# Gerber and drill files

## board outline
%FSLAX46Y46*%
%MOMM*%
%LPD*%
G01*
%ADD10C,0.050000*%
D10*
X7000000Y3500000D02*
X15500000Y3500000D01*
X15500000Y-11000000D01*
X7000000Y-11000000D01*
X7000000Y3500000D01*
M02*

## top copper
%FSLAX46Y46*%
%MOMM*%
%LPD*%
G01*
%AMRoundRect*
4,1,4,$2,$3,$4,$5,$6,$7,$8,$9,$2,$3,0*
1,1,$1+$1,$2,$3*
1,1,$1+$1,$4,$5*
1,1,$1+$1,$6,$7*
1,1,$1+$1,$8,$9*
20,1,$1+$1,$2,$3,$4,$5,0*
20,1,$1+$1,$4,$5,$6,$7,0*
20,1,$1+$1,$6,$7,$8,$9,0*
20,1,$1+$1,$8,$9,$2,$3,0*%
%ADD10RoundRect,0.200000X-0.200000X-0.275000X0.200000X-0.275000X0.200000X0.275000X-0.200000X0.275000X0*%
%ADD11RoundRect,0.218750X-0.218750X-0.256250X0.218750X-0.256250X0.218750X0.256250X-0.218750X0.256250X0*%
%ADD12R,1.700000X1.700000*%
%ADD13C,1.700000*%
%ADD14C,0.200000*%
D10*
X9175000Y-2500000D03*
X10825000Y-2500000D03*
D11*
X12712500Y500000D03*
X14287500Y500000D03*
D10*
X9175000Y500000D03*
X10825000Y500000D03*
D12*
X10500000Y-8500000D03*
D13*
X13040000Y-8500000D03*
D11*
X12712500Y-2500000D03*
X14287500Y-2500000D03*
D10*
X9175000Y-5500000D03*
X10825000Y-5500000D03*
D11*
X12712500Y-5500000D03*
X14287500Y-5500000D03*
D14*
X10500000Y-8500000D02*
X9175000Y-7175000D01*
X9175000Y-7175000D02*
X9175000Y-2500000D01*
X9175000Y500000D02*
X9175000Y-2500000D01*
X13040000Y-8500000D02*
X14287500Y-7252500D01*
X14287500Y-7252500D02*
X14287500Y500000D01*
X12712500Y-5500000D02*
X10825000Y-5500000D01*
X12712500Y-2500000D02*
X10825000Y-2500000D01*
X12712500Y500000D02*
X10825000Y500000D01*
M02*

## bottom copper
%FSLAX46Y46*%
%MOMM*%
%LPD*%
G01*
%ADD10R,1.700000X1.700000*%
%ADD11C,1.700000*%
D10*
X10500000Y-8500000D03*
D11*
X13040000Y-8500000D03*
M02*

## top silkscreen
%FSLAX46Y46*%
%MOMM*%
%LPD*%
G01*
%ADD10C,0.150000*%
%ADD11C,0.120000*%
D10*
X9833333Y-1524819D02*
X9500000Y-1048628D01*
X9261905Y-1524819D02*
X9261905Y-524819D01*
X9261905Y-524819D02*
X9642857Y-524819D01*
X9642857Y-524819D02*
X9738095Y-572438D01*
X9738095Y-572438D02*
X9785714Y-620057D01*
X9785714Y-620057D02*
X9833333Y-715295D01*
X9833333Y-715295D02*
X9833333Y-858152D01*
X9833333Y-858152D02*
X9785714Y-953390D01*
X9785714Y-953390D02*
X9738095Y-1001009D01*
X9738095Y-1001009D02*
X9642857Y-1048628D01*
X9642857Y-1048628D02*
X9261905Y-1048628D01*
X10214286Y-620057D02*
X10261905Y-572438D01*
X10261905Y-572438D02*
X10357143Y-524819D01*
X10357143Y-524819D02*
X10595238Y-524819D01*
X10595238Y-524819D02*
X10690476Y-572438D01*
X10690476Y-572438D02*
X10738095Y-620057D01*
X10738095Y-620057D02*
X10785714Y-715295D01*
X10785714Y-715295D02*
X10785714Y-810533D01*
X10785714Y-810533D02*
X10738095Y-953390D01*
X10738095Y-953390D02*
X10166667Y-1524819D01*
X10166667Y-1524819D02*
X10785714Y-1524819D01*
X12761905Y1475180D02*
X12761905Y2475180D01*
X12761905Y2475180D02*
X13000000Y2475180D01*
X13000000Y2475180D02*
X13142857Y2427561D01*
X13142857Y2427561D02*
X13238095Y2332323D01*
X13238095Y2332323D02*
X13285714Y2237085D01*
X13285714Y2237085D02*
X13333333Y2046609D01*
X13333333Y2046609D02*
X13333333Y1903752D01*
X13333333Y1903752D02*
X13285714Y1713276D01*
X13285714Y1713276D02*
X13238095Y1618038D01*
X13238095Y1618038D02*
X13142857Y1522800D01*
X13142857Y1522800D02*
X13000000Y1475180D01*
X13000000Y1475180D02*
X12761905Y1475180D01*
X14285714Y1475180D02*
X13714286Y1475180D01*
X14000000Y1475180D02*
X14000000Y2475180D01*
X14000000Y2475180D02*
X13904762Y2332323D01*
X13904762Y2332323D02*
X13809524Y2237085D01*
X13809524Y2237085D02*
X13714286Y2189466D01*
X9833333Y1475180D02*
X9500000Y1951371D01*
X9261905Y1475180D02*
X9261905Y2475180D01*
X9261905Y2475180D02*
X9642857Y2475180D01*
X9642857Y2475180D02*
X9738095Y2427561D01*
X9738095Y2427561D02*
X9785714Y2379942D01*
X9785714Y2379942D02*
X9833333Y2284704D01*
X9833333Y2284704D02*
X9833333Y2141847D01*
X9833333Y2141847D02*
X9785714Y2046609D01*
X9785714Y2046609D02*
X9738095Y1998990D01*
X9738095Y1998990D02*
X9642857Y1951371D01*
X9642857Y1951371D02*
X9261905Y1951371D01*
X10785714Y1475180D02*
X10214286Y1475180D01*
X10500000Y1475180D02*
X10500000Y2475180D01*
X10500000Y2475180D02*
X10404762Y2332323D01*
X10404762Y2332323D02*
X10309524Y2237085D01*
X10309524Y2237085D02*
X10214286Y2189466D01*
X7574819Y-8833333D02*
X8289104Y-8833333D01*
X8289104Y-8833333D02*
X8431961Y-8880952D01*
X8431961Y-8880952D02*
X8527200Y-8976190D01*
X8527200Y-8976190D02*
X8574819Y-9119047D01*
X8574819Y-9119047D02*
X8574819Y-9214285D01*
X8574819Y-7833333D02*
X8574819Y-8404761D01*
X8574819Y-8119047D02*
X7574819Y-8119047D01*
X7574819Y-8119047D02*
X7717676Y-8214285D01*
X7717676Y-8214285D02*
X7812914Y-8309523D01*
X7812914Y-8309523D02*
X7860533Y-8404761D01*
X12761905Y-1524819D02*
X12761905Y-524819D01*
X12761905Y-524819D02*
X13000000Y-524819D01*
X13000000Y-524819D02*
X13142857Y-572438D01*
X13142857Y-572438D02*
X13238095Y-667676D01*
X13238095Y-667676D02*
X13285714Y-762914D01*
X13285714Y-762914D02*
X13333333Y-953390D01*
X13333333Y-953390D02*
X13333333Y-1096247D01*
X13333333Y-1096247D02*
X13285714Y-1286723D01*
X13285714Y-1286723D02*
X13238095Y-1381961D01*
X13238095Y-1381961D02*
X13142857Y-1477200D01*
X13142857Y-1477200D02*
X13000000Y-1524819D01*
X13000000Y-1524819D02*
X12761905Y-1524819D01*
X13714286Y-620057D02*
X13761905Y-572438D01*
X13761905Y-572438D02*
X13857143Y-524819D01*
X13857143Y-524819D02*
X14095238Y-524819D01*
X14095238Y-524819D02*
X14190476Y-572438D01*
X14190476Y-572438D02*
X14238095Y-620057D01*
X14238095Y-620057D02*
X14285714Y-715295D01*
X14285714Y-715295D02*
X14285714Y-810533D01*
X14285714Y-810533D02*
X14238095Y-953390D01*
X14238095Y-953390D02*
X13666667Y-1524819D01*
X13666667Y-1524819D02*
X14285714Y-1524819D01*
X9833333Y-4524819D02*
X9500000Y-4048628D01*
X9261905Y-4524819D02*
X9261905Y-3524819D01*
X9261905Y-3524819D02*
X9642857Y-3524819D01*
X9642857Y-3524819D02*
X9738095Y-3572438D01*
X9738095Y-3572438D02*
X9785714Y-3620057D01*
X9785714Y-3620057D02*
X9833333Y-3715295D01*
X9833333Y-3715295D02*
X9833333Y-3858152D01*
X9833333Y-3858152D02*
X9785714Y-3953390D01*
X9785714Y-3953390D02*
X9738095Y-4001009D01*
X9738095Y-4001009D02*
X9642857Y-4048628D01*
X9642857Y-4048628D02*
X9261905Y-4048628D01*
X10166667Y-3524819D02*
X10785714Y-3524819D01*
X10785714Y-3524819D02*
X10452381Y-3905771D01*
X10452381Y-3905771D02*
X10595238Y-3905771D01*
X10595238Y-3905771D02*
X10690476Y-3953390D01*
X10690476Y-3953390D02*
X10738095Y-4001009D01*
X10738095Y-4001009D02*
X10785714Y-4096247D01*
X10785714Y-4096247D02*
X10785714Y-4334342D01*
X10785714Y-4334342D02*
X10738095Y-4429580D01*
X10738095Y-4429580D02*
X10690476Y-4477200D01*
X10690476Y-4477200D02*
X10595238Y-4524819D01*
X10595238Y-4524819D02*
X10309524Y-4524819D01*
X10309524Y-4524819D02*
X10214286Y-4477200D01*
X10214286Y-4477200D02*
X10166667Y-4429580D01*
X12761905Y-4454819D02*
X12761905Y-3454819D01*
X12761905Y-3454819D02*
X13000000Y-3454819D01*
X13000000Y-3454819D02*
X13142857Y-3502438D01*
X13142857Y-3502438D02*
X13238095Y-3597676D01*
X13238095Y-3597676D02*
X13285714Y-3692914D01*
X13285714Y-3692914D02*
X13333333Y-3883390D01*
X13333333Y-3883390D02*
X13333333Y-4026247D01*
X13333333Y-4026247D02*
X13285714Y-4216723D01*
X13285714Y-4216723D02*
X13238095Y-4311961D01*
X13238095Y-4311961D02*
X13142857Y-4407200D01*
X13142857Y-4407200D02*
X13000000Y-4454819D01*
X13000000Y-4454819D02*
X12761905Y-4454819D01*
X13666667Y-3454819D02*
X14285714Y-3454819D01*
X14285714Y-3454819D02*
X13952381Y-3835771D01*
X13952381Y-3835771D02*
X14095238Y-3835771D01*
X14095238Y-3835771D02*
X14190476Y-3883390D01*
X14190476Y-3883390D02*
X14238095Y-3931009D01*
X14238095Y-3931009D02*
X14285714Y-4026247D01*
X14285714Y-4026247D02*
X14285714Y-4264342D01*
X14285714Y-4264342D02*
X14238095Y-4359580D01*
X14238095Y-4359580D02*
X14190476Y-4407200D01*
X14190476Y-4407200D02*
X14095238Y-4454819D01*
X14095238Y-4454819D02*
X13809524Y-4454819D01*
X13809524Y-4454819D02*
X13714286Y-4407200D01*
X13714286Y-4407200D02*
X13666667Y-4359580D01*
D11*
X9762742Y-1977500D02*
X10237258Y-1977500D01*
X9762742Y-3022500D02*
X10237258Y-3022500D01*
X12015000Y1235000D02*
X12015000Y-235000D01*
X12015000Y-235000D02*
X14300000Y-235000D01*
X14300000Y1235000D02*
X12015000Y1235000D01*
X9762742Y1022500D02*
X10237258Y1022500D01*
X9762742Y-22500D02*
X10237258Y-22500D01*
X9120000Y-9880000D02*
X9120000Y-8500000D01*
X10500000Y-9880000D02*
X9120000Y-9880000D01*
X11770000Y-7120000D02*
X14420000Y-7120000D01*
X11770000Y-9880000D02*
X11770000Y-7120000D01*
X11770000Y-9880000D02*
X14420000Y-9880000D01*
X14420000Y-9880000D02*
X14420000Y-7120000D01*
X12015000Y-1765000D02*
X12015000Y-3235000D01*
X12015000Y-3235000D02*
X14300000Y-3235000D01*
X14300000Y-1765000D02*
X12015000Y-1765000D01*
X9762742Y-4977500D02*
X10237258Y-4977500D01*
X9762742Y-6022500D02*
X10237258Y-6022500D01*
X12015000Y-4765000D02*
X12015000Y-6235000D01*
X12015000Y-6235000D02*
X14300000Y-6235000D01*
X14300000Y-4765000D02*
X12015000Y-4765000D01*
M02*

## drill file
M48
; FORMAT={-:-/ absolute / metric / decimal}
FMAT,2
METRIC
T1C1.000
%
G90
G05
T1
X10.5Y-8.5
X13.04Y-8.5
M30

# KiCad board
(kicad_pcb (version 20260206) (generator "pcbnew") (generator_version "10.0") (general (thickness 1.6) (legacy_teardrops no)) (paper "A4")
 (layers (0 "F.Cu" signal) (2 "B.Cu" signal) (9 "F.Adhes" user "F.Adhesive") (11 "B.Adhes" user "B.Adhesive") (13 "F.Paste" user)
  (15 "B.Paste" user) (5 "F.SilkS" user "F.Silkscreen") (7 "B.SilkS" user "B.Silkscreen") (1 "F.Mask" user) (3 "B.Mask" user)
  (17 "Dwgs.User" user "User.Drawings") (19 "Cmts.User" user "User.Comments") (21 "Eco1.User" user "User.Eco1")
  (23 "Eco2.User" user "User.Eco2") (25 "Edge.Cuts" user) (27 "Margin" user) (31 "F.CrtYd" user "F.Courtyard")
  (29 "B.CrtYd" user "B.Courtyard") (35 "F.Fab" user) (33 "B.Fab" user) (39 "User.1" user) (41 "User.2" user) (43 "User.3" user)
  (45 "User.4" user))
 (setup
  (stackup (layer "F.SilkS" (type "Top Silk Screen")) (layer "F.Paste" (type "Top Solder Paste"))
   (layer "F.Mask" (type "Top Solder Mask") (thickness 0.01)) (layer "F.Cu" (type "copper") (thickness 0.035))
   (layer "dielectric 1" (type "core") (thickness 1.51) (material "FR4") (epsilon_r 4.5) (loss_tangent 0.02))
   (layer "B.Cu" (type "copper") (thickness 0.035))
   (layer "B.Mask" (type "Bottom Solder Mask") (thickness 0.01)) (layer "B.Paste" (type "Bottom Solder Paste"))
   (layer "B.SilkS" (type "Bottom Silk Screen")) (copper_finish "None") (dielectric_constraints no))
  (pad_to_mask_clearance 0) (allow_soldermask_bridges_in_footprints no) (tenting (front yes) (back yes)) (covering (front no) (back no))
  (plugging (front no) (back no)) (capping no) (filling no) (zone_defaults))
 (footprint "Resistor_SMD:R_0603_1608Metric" (layer "F.Cu") (at 10 2.5)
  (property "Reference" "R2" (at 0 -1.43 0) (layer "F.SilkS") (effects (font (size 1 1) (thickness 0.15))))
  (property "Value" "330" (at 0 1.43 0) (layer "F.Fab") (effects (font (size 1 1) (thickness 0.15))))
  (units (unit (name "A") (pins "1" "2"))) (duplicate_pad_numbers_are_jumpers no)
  (fp_line (start -0.237258 -0.5225) (end 0.237258 -0.5225) (stroke (width 0.12) (type solid)) (layer "F.SilkS"))
  (fp_line (start -0.237258 0.5225) (end 0.237258 0.5225) (stroke (width 0.12) (type solid)) (layer "F.SilkS"))
  (pad "1" smd roundrect (at -0.825 0) (size 0.8 0.95) (layers "F.Cu" "F.Mask" "F.Paste") (roundrect_rratio 0.25) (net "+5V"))
  (pad "2" smd roundrect (at 0.825 0) (size 0.8 0.95) (layers "F.Cu" "F.Mask" "F.Paste") (roundrect_rratio 0.25) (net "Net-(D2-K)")))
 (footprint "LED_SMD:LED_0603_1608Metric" (layer "F.Cu") (at 13.5 -0.5)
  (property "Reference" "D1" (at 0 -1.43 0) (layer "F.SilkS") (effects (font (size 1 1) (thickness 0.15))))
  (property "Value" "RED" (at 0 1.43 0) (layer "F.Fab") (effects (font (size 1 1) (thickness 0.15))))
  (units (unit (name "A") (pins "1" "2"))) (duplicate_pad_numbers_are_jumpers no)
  (fp_line (start -1.485 -0.735) (end -1.485 0.735) (stroke (width 0.12) (type solid)) (layer "F.SilkS"))
  (fp_line (start -1.485 0.735) (end 0.8 0.735) (stroke (width 0.12) (type solid)) (layer "F.SilkS"))
  (fp_line (start 0.8 -0.735) (end -1.485 -0.735) (stroke (width 0.12) (type solid)) (layer "F.SilkS"))
  (pad "1" smd roundrect (at -0.7875 0) (size 0.875 0.95) (layers "F.Cu" "F.Mask" "F.Paste") (roundrect_rratio 0.25) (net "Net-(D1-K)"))
  (pad "2" smd roundrect (at 0.7875 0) (size 0.875 0.95) (layers "F.Cu" "F.Mask" "F.Paste") (roundrect_rratio 0.25) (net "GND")))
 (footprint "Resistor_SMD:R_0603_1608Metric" (layer "F.Cu") (at 10 -0.5)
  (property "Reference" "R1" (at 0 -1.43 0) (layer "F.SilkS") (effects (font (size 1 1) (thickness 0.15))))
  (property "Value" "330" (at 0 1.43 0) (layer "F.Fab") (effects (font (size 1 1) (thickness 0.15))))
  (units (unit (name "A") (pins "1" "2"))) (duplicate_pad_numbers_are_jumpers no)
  (fp_line (start -0.237258 -0.5225) (end 0.237258 -0.5225) (stroke (width 0.12) (type solid)) (layer "F.SilkS"))
  (fp_line (start -0.237258 0.5225) (end 0.237258 0.5225) (stroke (width 0.12) (type solid)) (layer "F.SilkS"))
  (pad "1" smd roundrect (at -0.825 0) (size 0.8 0.95) (layers "F.Cu" "F.Mask" "F.Paste") (roundrect_rratio 0.25) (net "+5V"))
  (pad "2" smd roundrect (at 0.825 0) (size 0.8 0.95) (layers "F.Cu" "F.Mask" "F.Paste") (roundrect_rratio 0.25) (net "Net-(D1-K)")))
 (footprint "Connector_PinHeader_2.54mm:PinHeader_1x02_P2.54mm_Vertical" (layer "F.Cu") (at 10.5 8.5 90)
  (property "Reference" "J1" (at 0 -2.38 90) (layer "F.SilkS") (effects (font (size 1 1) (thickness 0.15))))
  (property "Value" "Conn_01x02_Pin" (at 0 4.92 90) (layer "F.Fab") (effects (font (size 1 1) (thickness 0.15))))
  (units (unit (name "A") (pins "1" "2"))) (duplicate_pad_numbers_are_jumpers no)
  (fp_line (start -1.38 -1.38) (end 0 -1.38) (stroke (width 0.12) (type solid)) (layer "F.SilkS"))
  (fp_line (start -1.38 0) (end -1.38 -1.38) (stroke (width 0.12) (type solid)) (layer "F.SilkS"))
  (fp_line (start 1.38 1.27) (end 1.38 3.92) (stroke (width 0.12) (type solid)) (layer "F.SilkS"))
  (fp_line (start -1.38 1.27) (end 1.38 1.27) (stroke (width 0.12) (type solid)) (layer "F.SilkS"))
  (fp_line (start -1.38 1.27) (end -1.38 3.92) (stroke (width 0.12) (type solid)) (layer "F.SilkS"))
  (fp_line (start -1.38 3.92) (end 1.38 3.92) (stroke (width 0.12) (type solid)) (layer "F.SilkS"))
  (pad "1" thru_hole rect (at 0 0 90) (size 1.7 1.7) (drill 1) (layers "*.Cu" "*.Mask") (remove_unused_layers no) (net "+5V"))
  (pad "2" thru_hole circle (at 0 2.54 90) (size 1.7 1.7) (drill 1) (layers "*.Cu" "*.Mask") (remove_unused_layers no) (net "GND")))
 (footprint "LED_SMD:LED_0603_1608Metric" (layer "F.Cu") (at 13.5 2.5)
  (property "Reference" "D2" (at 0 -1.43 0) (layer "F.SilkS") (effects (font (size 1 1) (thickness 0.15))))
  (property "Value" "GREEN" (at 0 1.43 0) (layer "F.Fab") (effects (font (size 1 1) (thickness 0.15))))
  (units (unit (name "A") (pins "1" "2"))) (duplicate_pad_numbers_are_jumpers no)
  (fp_line (start -1.485 -0.735) (end -1.485 0.735) (stroke (width 0.12) (type solid)) (layer "F.SilkS"))
  (fp_line (start -1.485 0.735) (end 0.8 0.735) (stroke (width 0.12) (type solid)) (layer "F.SilkS"))
  (fp_line (start 0.8 -0.735) (end -1.485 -0.735) (stroke (width 0.12) (type solid)) (layer "F.SilkS"))
  (pad "1" smd roundrect (at -0.7875 0) (size 0.875 0.95) (layers "F.Cu" "F.Mask" "F.Paste") (roundrect_rratio 0.25) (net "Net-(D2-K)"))
  (pad "2" smd roundrect (at 0.7875 0) (size 0.875 0.95) (layers "F.Cu" "F.Mask" "F.Paste") (roundrect_rratio 0.25) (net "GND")))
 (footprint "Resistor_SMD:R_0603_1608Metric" (layer "F.Cu") (at 10 5.5)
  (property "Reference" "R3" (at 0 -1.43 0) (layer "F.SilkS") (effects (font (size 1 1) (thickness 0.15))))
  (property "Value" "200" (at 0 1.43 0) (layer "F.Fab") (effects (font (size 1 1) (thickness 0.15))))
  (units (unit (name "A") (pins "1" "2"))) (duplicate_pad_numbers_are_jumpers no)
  (fp_line (start -0.237258 -0.5225) (end 0.237258 -0.5225) (stroke (width 0.12) (type solid)) (layer "F.SilkS"))
  (fp_line (start -0.237258 0.5225) (end 0.237258 0.5225) (stroke (width 0.12) (type solid)) (layer "F.SilkS"))
  (pad "1" smd roundrect (at -0.825 0) (size 0.8 0.95) (layers "F.Cu" "F.Mask" "F.Paste") (roundrect_rratio 0.25) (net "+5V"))
  (pad "2" smd roundrect (at 0.825 0) (size 0.8 0.95) (layers "F.Cu" "F.Mask" "F.Paste") (roundrect_rratio 0.25) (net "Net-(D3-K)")))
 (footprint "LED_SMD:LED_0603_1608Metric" (layer "F.Cu") (at 13.5 5.5)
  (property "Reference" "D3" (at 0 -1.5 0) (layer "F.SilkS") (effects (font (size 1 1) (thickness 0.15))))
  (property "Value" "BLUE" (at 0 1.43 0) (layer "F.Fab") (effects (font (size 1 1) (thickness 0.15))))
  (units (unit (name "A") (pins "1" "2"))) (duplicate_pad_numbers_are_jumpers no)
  (fp_line (start -1.485 -0.735) (end -1.485 0.735) (stroke (width 0.12) (type solid)) (layer "F.SilkS"))
  (fp_line (start -1.485 0.735) (end 0.8 0.735) (stroke (width 0.12) (type solid)) (layer "F.SilkS"))
  (fp_line (start 0.8 -0.735) (end -1.485 -0.735) (stroke (width 0.12) (type solid)) (layer "F.SilkS"))
  (pad "1" smd roundrect (at -0.7875 0) (size 0.875 0.95) (layers "F.Cu" "F.Mask" "F.Paste") (roundrect_rratio 0.25) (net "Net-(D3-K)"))
  (pad "2" smd roundrect (at 0.7875 0) (size 0.875 0.95) (layers "F.Cu" "F.Mask" "F.Paste") (roundrect_rratio 0.25) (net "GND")))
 (gr_rect (start 7 -3.5) (end 15.5 11) (stroke (width 0.05) (type default)) (fill no) (layer "Edge.Cuts"))
 (segment (start 10.5 8.5) (end 9.175 7.175) (width 0.2) (layer "F.Cu") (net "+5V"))
 (segment (start 9.175 7.175) (end 9.175 2.5) (width 0.2) (layer "F.Cu") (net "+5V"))
 (segment (start 9.175 -0.5) (end 9.175 2.5) (width 0.2) (layer "F.Cu") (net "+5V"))
 (segment (start 13.04 8.5) (end 14.2875 7.2525) (width 0.2) (layer "F.Cu") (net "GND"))
 (segment (start 14.2875 7.2525) (end 14.2875 -0.5) (width 0.2) (layer "F.Cu") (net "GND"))
 (segment (start 12.7125 5.5) (end 10.825 5.5) (width 0.2) (layer "F.Cu") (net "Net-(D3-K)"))
 (segment (start 12.7125 2.5) (end 10.825 2.5) (width 0.2) (layer "F.Cu") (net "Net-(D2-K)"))
 (segment (start 12.7125 -0.5) (end 10.825 -0.5) (width 0.2) (layer "F.Cu") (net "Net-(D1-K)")))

